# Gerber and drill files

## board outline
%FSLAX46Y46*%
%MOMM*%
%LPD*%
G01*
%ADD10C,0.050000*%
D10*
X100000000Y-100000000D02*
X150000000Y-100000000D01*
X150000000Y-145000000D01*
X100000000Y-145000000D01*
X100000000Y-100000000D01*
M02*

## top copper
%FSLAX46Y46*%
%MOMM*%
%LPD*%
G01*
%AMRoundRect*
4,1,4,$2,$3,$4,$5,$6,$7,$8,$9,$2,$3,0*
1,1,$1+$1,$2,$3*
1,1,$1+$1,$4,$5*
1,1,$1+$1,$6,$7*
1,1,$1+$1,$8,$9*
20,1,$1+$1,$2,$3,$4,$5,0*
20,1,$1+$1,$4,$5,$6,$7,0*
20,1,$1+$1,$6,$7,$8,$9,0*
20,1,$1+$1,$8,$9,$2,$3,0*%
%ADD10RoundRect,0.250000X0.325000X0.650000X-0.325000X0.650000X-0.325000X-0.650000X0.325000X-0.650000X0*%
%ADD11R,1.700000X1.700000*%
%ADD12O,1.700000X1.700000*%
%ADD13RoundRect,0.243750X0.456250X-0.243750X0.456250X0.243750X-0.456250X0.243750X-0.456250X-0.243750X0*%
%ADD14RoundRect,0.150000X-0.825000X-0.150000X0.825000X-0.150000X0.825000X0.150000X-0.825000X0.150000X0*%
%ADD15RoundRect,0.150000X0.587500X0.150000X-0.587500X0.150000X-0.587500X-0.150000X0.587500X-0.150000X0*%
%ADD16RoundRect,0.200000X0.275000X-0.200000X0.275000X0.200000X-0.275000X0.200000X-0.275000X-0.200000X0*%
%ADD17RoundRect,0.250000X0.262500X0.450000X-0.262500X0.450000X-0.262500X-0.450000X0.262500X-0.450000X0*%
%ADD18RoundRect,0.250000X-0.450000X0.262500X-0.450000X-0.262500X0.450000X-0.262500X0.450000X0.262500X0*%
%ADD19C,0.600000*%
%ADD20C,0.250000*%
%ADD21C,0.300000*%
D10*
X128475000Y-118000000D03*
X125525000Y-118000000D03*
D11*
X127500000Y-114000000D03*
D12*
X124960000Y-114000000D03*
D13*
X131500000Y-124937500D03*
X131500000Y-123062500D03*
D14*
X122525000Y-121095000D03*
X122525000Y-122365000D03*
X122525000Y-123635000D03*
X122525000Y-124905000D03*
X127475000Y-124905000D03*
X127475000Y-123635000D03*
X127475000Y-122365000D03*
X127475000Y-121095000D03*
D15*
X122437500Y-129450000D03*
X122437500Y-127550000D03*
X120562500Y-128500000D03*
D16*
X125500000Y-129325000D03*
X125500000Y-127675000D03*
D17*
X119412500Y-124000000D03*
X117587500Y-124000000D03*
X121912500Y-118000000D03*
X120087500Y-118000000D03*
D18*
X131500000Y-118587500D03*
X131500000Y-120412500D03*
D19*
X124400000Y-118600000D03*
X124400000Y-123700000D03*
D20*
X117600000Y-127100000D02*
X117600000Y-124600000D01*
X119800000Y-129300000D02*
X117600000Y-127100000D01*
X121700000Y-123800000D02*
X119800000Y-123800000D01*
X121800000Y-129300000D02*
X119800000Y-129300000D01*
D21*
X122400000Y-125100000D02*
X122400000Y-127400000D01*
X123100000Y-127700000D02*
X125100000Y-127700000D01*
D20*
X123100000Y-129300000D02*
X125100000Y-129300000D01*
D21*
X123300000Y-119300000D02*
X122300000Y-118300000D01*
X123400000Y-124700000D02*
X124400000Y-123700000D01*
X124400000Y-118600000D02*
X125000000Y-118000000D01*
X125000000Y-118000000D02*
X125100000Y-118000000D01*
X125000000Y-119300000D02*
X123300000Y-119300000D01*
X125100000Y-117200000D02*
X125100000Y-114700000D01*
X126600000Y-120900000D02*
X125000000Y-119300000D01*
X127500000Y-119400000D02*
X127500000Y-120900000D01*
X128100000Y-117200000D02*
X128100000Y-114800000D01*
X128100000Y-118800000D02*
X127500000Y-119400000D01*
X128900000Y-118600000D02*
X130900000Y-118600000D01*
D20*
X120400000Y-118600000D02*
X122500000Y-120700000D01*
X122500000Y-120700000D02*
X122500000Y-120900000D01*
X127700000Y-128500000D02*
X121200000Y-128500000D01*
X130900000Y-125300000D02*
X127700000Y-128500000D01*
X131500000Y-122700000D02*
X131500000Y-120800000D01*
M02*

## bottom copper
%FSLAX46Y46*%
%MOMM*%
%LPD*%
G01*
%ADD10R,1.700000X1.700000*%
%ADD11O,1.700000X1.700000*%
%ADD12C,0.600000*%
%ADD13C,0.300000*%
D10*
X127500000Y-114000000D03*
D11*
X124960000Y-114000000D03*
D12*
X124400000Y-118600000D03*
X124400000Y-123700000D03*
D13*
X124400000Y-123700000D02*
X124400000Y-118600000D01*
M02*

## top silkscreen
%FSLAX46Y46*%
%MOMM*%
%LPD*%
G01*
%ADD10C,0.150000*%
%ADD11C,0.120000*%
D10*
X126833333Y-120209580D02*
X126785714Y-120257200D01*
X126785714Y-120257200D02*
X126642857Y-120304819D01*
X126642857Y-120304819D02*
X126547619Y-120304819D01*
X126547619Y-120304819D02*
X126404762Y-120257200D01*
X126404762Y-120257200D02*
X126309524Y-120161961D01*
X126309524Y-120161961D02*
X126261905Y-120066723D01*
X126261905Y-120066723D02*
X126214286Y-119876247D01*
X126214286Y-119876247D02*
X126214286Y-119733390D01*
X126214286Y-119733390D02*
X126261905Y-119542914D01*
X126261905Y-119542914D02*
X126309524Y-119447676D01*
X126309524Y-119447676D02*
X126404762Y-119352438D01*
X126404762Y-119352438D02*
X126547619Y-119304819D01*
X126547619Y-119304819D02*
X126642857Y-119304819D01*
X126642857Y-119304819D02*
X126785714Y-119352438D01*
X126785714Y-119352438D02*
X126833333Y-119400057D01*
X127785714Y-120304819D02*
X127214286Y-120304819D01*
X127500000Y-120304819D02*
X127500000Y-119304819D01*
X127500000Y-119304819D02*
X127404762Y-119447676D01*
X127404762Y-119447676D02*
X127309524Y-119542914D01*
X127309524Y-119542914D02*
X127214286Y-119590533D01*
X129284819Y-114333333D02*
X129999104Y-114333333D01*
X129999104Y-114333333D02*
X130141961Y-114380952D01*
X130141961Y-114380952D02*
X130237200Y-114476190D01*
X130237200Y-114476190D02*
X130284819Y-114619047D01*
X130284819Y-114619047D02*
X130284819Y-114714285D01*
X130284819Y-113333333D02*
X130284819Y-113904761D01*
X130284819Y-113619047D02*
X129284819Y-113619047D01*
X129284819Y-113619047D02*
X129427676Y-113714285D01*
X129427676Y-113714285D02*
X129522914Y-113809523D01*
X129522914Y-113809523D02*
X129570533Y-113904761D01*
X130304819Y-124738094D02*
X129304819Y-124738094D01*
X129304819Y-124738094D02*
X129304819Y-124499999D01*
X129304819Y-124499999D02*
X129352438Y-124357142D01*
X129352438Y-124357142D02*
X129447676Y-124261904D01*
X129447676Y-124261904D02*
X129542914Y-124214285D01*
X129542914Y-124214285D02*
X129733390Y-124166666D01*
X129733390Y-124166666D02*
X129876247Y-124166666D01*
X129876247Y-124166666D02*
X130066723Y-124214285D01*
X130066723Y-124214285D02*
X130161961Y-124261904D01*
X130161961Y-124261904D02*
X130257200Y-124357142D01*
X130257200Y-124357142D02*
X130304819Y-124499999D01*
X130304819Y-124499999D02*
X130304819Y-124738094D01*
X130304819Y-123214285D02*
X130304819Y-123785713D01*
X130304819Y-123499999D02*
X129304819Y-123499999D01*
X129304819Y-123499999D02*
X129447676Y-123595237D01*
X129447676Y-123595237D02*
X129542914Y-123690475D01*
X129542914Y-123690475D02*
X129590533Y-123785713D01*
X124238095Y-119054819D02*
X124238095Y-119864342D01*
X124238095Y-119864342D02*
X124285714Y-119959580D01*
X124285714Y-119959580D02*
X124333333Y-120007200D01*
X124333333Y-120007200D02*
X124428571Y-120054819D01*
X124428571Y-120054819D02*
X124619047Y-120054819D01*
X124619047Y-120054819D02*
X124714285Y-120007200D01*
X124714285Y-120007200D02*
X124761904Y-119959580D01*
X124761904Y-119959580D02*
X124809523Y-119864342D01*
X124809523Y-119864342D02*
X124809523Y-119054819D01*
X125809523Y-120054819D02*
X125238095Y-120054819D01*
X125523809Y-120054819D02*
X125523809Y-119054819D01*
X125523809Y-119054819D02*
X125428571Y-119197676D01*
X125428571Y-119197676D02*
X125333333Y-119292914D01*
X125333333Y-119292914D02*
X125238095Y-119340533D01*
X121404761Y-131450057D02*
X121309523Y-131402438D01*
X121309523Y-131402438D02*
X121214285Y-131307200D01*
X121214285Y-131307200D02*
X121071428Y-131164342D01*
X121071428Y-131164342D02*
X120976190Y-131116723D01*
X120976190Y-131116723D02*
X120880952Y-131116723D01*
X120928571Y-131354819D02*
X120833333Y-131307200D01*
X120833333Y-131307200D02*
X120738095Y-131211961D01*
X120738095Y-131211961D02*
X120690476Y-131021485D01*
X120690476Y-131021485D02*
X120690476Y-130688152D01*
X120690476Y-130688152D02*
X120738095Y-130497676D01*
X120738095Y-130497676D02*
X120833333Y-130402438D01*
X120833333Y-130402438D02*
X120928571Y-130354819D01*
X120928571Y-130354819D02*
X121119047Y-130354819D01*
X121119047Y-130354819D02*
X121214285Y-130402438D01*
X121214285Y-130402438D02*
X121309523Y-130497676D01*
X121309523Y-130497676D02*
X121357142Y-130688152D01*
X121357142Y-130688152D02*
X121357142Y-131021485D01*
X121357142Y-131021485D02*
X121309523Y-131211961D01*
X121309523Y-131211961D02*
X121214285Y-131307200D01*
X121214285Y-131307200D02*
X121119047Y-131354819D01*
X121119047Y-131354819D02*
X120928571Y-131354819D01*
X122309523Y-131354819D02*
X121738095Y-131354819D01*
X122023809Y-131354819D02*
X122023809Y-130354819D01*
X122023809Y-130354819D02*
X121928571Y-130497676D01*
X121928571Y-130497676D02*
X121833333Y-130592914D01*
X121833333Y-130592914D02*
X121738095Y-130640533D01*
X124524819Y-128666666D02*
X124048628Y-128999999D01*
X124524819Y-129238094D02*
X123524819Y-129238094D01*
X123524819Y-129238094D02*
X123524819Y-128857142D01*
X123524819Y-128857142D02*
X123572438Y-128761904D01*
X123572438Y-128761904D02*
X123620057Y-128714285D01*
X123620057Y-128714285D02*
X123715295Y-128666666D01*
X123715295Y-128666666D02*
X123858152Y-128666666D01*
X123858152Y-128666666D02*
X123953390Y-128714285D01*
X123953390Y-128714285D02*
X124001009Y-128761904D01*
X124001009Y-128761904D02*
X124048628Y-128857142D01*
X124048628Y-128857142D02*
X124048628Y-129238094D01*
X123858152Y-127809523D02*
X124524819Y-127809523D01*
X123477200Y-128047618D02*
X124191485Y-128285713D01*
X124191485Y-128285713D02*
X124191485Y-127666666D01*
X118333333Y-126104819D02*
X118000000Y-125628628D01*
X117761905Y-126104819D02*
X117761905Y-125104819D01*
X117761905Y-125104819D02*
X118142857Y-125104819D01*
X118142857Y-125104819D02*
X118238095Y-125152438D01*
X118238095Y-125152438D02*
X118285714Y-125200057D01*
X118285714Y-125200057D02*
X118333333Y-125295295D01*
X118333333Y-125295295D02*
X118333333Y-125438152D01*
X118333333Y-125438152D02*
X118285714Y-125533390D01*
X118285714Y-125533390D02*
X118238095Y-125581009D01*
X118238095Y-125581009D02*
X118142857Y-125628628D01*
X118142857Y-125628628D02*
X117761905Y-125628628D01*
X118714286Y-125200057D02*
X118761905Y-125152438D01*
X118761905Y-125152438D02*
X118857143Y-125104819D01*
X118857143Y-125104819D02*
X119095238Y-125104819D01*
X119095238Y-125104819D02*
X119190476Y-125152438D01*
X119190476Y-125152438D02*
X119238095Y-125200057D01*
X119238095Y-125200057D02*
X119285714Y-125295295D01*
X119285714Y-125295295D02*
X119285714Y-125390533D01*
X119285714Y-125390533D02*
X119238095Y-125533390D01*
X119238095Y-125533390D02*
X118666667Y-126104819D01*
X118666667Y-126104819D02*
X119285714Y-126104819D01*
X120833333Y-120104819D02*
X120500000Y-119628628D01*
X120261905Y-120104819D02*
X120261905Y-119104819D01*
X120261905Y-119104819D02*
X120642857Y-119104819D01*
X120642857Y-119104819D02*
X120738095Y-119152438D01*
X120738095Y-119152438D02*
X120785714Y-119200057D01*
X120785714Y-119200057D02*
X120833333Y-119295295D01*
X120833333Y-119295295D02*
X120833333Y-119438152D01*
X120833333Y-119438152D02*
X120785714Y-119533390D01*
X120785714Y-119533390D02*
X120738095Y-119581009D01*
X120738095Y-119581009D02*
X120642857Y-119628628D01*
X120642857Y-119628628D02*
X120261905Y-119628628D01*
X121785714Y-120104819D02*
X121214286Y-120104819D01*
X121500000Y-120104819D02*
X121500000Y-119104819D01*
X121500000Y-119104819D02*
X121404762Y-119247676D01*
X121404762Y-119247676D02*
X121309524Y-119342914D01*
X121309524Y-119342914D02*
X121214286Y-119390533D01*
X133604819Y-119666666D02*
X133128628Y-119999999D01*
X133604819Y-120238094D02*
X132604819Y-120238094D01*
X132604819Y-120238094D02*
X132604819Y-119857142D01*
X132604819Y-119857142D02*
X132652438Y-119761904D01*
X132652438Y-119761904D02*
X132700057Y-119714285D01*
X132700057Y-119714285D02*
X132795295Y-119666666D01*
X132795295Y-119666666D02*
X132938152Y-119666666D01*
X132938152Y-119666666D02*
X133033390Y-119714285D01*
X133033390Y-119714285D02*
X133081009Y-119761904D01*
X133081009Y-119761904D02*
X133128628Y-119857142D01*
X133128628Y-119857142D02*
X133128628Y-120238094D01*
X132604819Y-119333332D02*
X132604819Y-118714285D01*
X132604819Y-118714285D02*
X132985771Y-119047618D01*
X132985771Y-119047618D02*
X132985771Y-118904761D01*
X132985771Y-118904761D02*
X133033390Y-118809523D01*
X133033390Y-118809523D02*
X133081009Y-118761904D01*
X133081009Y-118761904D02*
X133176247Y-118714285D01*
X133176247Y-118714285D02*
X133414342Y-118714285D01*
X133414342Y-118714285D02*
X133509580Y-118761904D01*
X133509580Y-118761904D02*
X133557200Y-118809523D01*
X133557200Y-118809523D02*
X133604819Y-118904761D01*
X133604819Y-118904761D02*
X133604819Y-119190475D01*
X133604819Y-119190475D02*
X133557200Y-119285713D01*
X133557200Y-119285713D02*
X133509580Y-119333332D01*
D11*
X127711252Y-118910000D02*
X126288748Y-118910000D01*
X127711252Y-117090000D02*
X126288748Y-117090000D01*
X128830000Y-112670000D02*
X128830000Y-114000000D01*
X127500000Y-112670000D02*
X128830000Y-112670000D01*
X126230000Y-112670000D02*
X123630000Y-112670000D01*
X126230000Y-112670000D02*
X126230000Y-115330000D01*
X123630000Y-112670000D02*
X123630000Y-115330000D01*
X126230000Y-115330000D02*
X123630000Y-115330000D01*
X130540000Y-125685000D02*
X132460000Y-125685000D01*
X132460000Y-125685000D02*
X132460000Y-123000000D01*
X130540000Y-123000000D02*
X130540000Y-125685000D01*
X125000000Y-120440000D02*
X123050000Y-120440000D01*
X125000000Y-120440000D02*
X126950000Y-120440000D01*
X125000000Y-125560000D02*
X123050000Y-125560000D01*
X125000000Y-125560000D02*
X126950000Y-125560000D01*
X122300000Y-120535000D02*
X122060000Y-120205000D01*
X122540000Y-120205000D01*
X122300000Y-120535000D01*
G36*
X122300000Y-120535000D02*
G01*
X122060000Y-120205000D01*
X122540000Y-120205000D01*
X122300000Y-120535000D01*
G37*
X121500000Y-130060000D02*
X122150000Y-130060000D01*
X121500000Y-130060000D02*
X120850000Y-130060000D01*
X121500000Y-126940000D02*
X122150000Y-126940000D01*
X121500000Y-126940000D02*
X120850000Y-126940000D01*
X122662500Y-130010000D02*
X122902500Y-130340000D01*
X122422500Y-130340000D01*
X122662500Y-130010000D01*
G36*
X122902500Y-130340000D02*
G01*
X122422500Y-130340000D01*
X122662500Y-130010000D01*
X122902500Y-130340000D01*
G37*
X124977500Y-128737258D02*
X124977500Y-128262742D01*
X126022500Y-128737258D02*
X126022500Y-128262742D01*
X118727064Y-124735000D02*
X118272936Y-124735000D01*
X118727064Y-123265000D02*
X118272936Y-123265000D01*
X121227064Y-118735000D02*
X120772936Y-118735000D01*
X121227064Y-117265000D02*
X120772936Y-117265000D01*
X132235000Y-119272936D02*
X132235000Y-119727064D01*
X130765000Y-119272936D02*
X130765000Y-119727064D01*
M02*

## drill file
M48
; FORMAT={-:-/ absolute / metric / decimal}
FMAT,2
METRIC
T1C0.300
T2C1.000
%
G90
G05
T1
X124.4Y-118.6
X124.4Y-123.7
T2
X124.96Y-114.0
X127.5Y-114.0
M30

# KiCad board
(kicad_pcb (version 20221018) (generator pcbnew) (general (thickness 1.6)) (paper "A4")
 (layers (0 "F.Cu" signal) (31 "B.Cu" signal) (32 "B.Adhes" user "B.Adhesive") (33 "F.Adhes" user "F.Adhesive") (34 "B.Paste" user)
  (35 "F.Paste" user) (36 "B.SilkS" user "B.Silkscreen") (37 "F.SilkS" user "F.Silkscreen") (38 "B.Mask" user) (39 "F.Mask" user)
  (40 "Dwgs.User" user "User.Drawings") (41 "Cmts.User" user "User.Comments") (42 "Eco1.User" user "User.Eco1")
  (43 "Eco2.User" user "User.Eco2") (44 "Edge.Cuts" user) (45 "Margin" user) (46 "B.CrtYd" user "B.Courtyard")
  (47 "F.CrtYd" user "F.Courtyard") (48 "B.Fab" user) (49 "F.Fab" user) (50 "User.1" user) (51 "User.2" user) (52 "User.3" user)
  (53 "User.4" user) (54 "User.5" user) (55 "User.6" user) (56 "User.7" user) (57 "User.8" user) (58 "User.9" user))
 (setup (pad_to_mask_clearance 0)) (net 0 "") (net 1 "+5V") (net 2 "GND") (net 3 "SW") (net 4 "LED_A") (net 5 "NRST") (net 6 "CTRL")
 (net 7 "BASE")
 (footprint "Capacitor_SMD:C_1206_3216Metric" (layer "F.Cu") (at 127 118 180)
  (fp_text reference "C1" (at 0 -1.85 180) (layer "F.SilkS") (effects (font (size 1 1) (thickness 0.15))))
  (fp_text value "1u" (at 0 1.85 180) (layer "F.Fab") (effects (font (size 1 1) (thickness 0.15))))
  (fp_line (start -0.711252 -0.91) (end 0.711252 -0.91) (stroke (width 0.12) (type solid)) (layer "F.SilkS"))
  (fp_line (start -0.711252 0.91) (end 0.711252 0.91) (stroke (width 0.12) (type solid)) (layer "F.SilkS"))
  (pad "1" smd roundrect (at -1.475 0 180) (size 1.15 1.8) (layers "F.Cu" "F.Paste" "F.Mask") (roundrect_rratio 0.217391) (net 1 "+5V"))
  (pad "2" smd roundrect (at 1.475 0 180) (size 1.15 1.8) (layers "F.Cu" "F.Paste" "F.Mask") (roundrect_rratio 0.217391) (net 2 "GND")))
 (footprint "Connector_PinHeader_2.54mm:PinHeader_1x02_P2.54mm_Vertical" (layer "F.Cu") (at 127.5 114 -90)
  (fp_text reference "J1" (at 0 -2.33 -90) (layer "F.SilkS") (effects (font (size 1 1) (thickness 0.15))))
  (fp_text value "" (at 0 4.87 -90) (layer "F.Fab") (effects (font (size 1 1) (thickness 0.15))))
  (fp_line (start -1.33 -1.33) (end 0 -1.33) (stroke (width 0.12) (type solid)) (layer "F.SilkS"))
  (fp_line (start -1.33 0) (end -1.33 -1.33) (stroke (width 0.12) (type solid)) (layer "F.SilkS"))
  (fp_line (start -1.33 1.27) (end -1.33 3.87) (stroke (width 0.12) (type solid)) (layer "F.SilkS"))
  (fp_line (start -1.33 1.27) (end 1.33 1.27) (stroke (width 0.12) (type solid)) (layer "F.SilkS"))
  (fp_line (start -1.33 3.87) (end 1.33 3.87) (stroke (width 0.12) (type solid)) (layer "F.SilkS"))
  (fp_line (start 1.33 1.27) (end 1.33 3.87) (stroke (width 0.12) (type solid)) (layer "F.SilkS"))
  (pad "1" thru_hole rect (at 0 0 270) (size 1.7 1.7) (drill 1) (layers "*.Cu" "*.Mask") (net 1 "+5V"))
  (pad "2" thru_hole oval (at 0 2.54 270) (size 1.7 1.7) (drill 1) (layers "*.Cu" "*.Mask") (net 2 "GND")))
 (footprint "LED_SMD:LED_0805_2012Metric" (layer "F.Cu") (at 131.5 124 90)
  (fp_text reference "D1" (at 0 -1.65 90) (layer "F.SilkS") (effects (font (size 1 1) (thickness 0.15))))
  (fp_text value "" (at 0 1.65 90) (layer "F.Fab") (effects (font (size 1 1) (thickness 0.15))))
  (fp_line (start -1.685 -0.96) (end -1.685 0.96) (stroke (width 0.12) (type solid)) (layer "F.SilkS"))
  (fp_line (start -1.685 0.96) (end 1 0.96) (stroke (width 0.12) (type solid)) (layer "F.SilkS"))
  (fp_line (start 1 -0.96) (end -1.685 -0.96) (stroke (width 0.12) (type solid)) (layer "F.SilkS"))
  (pad "1" smd roundrect (at -0.9375 0 90) (size 0.975 1.4) (layers "F.Cu" "F.Paste" "F.Mask") (roundrect_rratio 0.25) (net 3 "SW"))
  (pad "2" smd roundrect (at 0.9375 0 90) (size 0.975 1.4) (layers "F.Cu" "F.Paste" "F.Mask") (roundrect_rratio 0.25) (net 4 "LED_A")))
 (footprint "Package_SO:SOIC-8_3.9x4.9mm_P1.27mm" (layer "F.Cu") (at 125 123)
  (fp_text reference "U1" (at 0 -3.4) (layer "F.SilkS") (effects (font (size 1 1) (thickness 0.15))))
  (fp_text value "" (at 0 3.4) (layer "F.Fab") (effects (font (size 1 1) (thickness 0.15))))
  (fp_line (start 0 -2.56) (end -1.95 -2.56) (stroke (width 0.12) (type solid)) (layer "F.SilkS"))
  (fp_line (start 0 -2.56) (end 1.95 -2.56) (stroke (width 0.12) (type solid)) (layer "F.SilkS"))
  (fp_line (start 0 2.56) (end -1.95 2.56) (stroke (width 0.12) (type solid)) (layer "F.SilkS"))
  (fp_line (start 0 2.56) (end 1.95 2.56) (stroke (width 0.12) (type solid)) (layer "F.SilkS"))
  (fp_poly
   (pts (xy -2.7 -2.465) (xy -2.94 -2.795) (xy -2.46 -2.795) (xy -2.7 -2.465)) (stroke (width 0.12) (type solid)) (fill solid)
   (layer "F.SilkS"))
  (pad "1" smd roundrect (at -2.475 -1.905) (size 1.95 0.6) (layers "F.Cu" "F.Paste" "F.Mask") (roundrect_rratio 0.25) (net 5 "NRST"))
  (pad "2" smd roundrect (at -2.475 -0.635) (size 1.95 0.6) (layers "F.Cu" "F.Paste" "F.Mask") (roundrect_rratio 0.25))
  (pad "3" smd roundrect (at -2.475 0.635) (size 1.95 0.6) (layers "F.Cu" "F.Paste" "F.Mask") (roundrect_rratio 0.25) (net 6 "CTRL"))
  (pad "4" smd roundrect (at -2.475 1.905) (size 1.95 0.6) (layers "F.Cu" "F.Paste" "F.Mask") (roundrect_rratio 0.25) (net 2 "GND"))
  (pad "5" smd roundrect (at 2.475 1.905) (size 1.95 0.6) (layers "F.Cu" "F.Paste" "F.Mask") (roundrect_rratio 0.25))
  (pad "6" smd roundrect (at 2.475 0.635) (size 1.95 0.6) (layers "F.Cu" "F.Paste" "F.Mask") (roundrect_rratio 0.25))
  (pad "7" smd roundrect (at 2.475 -0.635) (size 1.95 0.6) (layers "F.Cu" "F.Paste" "F.Mask") (roundrect_rratio 0.25))
  (pad "8" smd roundrect (at 2.475 -1.905) (size 1.95 0.6) (layers "F.Cu" "F.Paste" "F.Mask") (roundrect_rratio 0.25) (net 1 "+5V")))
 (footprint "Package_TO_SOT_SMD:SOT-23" (layer "F.Cu") (at 121.5 128.5 180)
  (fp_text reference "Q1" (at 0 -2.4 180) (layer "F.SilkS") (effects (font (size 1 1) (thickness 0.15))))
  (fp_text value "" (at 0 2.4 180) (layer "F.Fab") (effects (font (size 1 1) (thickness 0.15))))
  (fp_line (start 0 -1.56) (end -0.65 -1.56) (stroke (width 0.12) (type solid)) (layer "F.SilkS"))
  (fp_line (start 0 -1.56) (end 0.65 -1.56) (stroke (width 0.12) (type solid)) (layer "F.SilkS"))
  (fp_line (start 0 1.56) (end -0.65 1.56) (stroke (width 0.12) (type solid)) (layer "F.SilkS"))
  (fp_line (start 0 1.56) (end 0.65 1.56) (stroke (width 0.12) (type solid)) (layer "F.SilkS"))
  (fp_poly
   (pts (xy -1.1625 -1.51) (xy -1.4025 -1.84) (xy -0.9225 -1.84) (xy -1.1625 -1.51)) (stroke (width 0.12) (type solid)) (fill solid)
   (layer "F.SilkS"))
  (pad "1" smd roundrect (at -0.9375 -0.95 180) (size 1.475 0.6) (layers "F.Cu" "F.Paste" "F.Mask") (roundrect_rratio 0.25) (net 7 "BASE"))
  (pad "2" smd roundrect (at -0.9375 0.95 180) (size 1.475 0.6) (layers "F.Cu" "F.Paste" "F.Mask") (roundrect_rratio 0.25) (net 2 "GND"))
  (pad "3" smd roundrect (at 0.9375 0 180) (size 1.475 0.6) (layers "F.Cu" "F.Paste" "F.Mask") (roundrect_rratio 0.25) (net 3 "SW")))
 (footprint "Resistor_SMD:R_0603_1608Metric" (layer "F.Cu") (at 125.5 128.5 90)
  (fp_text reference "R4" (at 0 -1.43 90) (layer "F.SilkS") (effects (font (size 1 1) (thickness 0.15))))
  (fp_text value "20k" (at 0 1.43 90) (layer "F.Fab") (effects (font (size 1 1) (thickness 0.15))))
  (fp_line (start -0.237258 -0.5225) (end 0.237258 -0.5225) (stroke (width 0.12) (type solid)) (layer "F.SilkS"))
  (fp_line (start -0.237258 0.5225) (end 0.237258 0.5225) (stroke (width 0.12) (type solid)) (layer "F.SilkS"))
  (pad "1" smd roundrect (at -0.825 0 90) (size 0.8 0.95) (layers "F.Cu" "F.Paste" "F.Mask") (roundrect_rratio 0.25) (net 7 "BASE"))
  (pad "2" smd roundrect (at 0.825 0 90) (size 0.8 0.95) (layers "F.Cu" "F.Paste" "F.Mask") (roundrect_rratio 0.25) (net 2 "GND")))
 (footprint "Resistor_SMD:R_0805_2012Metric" (layer "F.Cu") (at 118.5 124 180)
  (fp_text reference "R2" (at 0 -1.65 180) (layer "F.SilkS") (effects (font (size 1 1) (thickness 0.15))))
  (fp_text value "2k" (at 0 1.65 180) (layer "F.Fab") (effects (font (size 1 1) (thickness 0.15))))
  (fp_line (start -0.227064 -0.735) (end 0.227064 -0.735) (stroke (width 0.12) (type solid)) (layer "F.SilkS"))
  (fp_line (start -0.227064 0.735) (end 0.227064 0.735) (stroke (width 0.12) (type solid)) (layer "F.SilkS"))
  (pad "1" smd roundrect (at -0.9125 0 180) (size 1.025 1.4) (layers "F.Cu" "F.Paste" "F.Mask") (roundrect_rratio 0.243902) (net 6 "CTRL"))
  (pad "2" smd roundrect (at 0.9125 0 180) (size 1.025 1.4) (layers "F.Cu" "F.Paste" "F.Mask") (roundrect_rratio 0.243902) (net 7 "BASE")))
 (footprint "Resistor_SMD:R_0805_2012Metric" (layer "F.Cu") (at 121 118 180)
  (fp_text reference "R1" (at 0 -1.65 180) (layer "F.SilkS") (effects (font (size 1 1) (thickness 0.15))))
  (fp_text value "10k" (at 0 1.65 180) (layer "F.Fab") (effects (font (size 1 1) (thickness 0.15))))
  (fp_line (start -0.227064 -0.735) (end 0.227064 -0.735) (stroke (width 0.12) (type solid)) (layer "F.SilkS"))
  (fp_line (start -0.227064 0.735) (end 0.227064 0.735) (stroke (width 0.12) (type solid)) (layer "F.SilkS"))
  (pad "1" smd roundrect (at -0.9125 0 180) (size 1.025 1.4) (layers "F.Cu" "F.Paste" "F.Mask") (roundrect_rratio 0.243902) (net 1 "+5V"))
  (pad "2" smd roundrect (at 0.9125 0 180) (size 1.025 1.4) (layers "F.Cu" "F.Paste" "F.Mask") (roundrect_rratio 0.243902) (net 5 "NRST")))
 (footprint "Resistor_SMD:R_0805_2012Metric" (layer "F.Cu") (at 131.5 119.5 -90)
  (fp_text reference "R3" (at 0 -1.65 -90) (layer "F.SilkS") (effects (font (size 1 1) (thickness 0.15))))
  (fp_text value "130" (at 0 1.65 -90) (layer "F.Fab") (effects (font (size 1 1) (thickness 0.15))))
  (fp_line (start -0.227064 -0.735) (end 0.227064 -0.735) (stroke (width 0.12) (type solid)) (layer "F.SilkS"))
  (fp_line (start -0.227064 0.735) (end 0.227064 0.735) (stroke (width 0.12) (type solid)) (layer "F.SilkS"))
  (pad "1" smd roundrect (at -0.9125 0 270) (size 1.025 1.4) (layers "F.Cu" "F.Paste" "F.Mask") (roundrect_rratio 0.243902) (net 1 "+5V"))
  (pad "2" smd roundrect (at 0.9125 0 270) (size 1.025 1.4) (layers "F.Cu" "F.Paste" "F.Mask") (roundrect_rratio 0.243902) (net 4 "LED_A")))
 (gr_rect (start 100 100) (end 150 145) (stroke (width 0.05) (type default)) (fill none) (layer "Edge.Cuts"))
 (segment (start 117.6 127.1) (end 117.6 124.6) (width 0.25) (layer "F.Cu") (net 7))
 (segment (start 119.8 129.3) (end 117.6 127.1) (width 0.25) (layer "F.Cu") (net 7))
 (segment (start 121.7 123.8) (end 119.8 123.8) (width 0.25) (layer "F.Cu") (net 6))
 (segment (start 121.8 129.3) (end 119.8 129.3) (width 0.25) (layer "F.Cu") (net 7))
 (segment (start 122.4 125.1) (end 122.4 127.4) (width 0.3) (layer "F.Cu") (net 2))
 (segment (start 123.1 127.7) (end 125.1 127.7) (width 0.3) (layer "F.Cu") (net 2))
 (segment (start 123.1 129.3) (end 125.1 129.3) (width 0.25) (layer "F.Cu") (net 7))
 (segment (start 123.3 119.3) (end 122.3 118.3) (width 0.3) (layer "F.Cu") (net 1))
 (segment (start 123.4 124.7) (end 124.4 123.7) (width 0.3) (layer "F.Cu") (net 2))
 (segment (start 124.4 118.6) (end 125 118) (width 0.3) (layer "F.Cu") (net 2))
 (segment (start 125 118) (end 125.1 118) (width 0.3) (layer "F.Cu") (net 2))
 (segment (start 125 119.3) (end 123.3 119.3) (width 0.3) (layer "F.Cu") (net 1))
 (segment (start 125.1 117.2) (end 125.1 114.7) (width 0.3) (layer "F.Cu") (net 2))
 (segment (start 126.6 120.9) (end 125 119.3) (width 0.3) (layer "F.Cu") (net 1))
 (segment (start 127.5 119.4) (end 127.5 120.9) (width 0.3) (layer "F.Cu") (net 1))
 (segment (start 128.1 117.2) (end 128.1 114.8) (width 0.3) (layer "F.Cu") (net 1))
 (segment (start 128.1 118.8) (end 127.5 119.4) (width 0.3) (layer "F.Cu") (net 1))
 (segment (start 128.9 118.6) (end 130.9 118.6) (width 0.3) (layer "F.Cu") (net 1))
 (via (at 124.4 118.6) (size 0.6) (drill 0.3) (layers "F.Cu" "B.Cu") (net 2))
 (via (at 124.4 123.7) (size 0.6) (drill 0.3) (layers "F.Cu" "B.Cu") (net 2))
 (segment (start 120.4 118.6) (end 122.5 120.7) (width 0.25) (layer "F.Cu") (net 5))
 (segment (start 122.5 120.7) (end 122.5 120.9) (width 0.25) (layer "F.Cu") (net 5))
 (segment (start 124.4 123.7) (end 124.4 118.6) (width 0.3) (layer "B.Cu") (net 2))
 (segment (start 127.7 128.5) (end 121.2 128.5) (width 0.25) (layer "F.Cu") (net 3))
 (segment (start 130.9 125.3) (end 127.7 128.5) (width 0.25) (layer "F.Cu") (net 3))
 (segment (start 131.5 122.7) (end 131.5 120.8) (width 0.25) (layer "F.Cu") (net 4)))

